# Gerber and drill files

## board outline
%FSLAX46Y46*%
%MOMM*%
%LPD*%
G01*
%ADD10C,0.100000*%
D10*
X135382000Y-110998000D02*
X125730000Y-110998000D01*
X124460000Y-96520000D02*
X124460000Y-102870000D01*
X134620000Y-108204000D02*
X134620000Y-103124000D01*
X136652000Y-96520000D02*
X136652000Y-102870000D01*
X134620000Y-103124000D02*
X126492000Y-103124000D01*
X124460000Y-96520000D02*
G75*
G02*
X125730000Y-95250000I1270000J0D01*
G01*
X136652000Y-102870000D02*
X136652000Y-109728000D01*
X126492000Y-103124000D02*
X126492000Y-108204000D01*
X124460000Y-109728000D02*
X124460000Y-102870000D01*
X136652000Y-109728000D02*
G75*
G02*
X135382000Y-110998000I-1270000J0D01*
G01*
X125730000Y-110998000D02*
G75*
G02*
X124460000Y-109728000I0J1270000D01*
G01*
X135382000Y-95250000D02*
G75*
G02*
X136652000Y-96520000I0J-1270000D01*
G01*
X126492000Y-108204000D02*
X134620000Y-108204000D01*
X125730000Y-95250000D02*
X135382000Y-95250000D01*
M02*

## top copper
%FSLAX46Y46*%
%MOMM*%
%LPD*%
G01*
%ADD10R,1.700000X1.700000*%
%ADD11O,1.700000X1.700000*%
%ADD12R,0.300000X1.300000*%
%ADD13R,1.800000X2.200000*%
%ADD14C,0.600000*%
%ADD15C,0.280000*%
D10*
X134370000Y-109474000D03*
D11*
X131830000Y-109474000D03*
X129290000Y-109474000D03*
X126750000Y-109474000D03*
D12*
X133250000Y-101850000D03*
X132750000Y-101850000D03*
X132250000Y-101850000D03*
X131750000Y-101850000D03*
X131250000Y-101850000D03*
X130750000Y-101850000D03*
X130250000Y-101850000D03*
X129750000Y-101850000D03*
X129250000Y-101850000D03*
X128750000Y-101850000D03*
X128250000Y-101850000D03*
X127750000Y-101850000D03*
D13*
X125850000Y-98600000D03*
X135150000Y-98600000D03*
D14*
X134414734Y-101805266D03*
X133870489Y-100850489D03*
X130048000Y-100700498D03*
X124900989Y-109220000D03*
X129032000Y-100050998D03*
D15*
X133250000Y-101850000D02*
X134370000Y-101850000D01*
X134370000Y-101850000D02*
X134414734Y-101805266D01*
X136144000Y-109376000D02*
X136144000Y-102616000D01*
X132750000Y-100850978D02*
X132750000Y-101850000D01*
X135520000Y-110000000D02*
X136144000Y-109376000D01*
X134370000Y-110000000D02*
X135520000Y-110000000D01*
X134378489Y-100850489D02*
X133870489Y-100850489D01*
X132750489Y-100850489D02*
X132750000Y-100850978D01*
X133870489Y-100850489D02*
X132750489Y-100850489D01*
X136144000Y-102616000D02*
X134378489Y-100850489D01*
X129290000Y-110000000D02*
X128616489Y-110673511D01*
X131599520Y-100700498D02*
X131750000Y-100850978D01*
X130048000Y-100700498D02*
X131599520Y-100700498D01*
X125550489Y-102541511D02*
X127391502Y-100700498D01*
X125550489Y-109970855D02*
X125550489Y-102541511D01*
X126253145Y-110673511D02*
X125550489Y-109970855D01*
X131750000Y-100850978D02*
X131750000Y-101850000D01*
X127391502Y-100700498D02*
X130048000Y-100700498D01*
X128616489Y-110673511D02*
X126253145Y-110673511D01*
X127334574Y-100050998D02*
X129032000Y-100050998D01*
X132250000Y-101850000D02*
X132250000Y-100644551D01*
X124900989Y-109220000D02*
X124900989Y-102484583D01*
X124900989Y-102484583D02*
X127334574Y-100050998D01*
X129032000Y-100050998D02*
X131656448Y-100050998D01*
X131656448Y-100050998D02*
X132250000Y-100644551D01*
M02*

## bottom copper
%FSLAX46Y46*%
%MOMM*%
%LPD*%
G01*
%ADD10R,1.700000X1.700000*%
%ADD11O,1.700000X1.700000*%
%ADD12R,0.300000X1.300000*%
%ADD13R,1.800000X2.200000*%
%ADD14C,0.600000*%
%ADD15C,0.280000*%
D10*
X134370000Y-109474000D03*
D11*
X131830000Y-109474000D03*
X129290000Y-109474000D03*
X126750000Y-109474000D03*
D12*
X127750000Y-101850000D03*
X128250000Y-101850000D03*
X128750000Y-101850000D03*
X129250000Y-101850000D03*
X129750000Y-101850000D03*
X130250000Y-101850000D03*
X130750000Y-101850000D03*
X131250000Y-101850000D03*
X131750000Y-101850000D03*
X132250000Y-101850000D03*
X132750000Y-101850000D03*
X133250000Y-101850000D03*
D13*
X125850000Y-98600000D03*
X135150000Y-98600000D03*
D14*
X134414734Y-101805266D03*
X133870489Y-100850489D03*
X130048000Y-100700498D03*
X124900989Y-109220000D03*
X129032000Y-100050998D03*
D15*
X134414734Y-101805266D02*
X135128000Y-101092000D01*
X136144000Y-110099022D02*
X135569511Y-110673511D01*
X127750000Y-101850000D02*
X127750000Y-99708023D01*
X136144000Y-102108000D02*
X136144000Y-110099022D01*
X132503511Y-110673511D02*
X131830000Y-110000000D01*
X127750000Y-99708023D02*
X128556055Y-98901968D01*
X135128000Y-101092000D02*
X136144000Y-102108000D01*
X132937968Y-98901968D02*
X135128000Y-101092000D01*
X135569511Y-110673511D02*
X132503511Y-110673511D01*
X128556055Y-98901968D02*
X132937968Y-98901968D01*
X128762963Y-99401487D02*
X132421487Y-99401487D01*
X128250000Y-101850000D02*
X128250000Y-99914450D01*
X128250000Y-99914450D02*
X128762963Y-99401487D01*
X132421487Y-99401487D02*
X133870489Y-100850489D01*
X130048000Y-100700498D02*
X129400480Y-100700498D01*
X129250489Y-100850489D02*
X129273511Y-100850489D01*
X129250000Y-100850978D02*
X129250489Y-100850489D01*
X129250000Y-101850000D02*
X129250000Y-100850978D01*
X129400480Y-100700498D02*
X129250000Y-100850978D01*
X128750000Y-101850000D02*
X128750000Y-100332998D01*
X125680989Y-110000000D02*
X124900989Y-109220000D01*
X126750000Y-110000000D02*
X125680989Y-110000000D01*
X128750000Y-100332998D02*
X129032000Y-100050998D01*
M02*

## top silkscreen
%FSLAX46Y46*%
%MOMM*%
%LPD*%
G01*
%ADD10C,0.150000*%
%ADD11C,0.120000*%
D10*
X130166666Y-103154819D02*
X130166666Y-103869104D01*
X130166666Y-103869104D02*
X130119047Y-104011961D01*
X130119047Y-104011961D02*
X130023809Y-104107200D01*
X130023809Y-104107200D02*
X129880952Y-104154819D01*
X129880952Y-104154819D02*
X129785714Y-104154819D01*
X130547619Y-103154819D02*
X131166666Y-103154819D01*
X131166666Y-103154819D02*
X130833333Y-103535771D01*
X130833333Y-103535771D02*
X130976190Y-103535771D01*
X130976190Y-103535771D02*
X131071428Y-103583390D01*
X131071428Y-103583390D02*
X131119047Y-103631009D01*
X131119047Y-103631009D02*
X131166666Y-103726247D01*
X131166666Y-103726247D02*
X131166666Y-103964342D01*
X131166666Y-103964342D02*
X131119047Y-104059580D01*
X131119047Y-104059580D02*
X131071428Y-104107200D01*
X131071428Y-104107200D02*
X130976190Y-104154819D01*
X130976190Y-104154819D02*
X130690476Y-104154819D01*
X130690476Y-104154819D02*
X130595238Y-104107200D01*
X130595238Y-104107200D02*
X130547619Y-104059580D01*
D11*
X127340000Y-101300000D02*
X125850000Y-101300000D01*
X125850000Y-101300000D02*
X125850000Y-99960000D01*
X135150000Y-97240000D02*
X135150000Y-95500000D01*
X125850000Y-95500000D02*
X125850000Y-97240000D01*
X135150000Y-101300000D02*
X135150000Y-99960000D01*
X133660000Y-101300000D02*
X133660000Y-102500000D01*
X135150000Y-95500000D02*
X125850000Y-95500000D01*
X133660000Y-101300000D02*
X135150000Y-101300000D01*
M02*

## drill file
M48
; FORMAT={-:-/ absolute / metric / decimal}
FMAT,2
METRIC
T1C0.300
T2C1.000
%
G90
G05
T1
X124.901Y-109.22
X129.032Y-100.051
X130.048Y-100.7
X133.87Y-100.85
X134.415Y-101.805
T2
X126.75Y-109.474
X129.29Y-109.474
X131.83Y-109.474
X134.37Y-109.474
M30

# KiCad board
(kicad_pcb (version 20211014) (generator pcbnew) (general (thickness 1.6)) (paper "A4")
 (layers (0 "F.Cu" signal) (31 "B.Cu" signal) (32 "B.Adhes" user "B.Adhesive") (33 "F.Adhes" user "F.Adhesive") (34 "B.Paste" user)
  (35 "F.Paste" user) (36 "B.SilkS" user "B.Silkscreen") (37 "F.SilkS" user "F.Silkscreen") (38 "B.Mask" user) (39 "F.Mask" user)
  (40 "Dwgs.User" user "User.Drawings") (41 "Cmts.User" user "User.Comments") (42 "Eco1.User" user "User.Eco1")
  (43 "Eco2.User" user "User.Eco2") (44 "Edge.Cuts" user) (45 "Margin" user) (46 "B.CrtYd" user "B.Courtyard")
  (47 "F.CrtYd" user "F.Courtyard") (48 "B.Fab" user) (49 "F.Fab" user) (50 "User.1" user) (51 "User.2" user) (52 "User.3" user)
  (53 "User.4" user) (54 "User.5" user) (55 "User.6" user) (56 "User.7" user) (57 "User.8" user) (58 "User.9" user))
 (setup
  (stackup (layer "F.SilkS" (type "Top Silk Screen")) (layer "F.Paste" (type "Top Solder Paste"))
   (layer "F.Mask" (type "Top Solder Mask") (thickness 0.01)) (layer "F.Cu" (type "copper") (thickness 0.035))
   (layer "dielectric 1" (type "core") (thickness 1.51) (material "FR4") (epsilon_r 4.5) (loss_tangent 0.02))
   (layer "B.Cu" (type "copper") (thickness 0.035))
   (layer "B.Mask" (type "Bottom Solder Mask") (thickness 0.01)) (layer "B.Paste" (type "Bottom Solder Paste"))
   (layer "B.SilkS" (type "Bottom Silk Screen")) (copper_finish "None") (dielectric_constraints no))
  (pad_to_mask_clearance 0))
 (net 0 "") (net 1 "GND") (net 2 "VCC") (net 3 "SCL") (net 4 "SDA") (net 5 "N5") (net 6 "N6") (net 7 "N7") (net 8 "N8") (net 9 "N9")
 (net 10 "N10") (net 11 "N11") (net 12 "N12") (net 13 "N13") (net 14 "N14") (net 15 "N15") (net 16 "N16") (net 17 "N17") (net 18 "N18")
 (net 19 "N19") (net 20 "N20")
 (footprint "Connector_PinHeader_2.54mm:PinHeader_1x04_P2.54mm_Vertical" (layer "F.Cu") (at 130.5 109.474 -90)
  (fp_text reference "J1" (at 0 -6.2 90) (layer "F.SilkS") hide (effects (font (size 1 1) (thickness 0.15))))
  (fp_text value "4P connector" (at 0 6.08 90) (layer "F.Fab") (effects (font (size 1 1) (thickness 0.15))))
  (pad "1" thru_hole rect (at 0 -3.87 270) (size 1.7 1.7) (drill 1) (layers *.Cu *.Mask) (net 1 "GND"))
  (pad "2" thru_hole oval (at 0 -1.33 270) (size 1.7 1.7) (drill 1) (layers *.Cu *.Mask) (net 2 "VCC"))
  (pad "3" thru_hole oval (at 0 1.21 270) (size 1.7 1.7) (drill 1) (layers *.Cu *.Mask) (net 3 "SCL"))
  (pad "4" thru_hole oval (at 0 3.75 270) (size 1.7 1.7) (drill 1) (layers *.Cu *.Mask) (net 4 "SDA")))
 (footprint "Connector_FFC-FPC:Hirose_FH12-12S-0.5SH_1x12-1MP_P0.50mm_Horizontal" (layer "F.Cu") (at 130.5 100 180)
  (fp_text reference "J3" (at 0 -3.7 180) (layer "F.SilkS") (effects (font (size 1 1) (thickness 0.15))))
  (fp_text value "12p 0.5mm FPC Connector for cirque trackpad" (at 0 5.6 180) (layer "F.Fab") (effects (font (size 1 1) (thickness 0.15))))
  (fp_line (start 3.16 -1.3) (end 4.65 -1.3) (layer "F.SilkS") (width 0.12))
  (fp_line (start 4.65 -1.3) (end 4.65 0.04) (layer "F.SilkS") (width 0.12))
  (fp_line (start -4.65 2.76) (end -4.65 4.5) (layer "F.SilkS") (width 0.12))
  (fp_line (start 4.65 4.5) (end 4.65 2.76) (layer "F.SilkS") (width 0.12))
  (fp_line (start -4.65 -1.3) (end -4.65 0.04) (layer "F.SilkS") (width 0.12))
  (fp_line (start -3.16 -1.3) (end -3.16 -2.5) (layer "F.SilkS") (width 0.12))
  (fp_line (start -4.65 4.5) (end 4.65 4.5) (layer "F.SilkS") (width 0.12))
  (fp_line (start -3.16 -1.3) (end -4.65 -1.3) (layer "F.SilkS") (width 0.12))
  (pad "1" smd rect (at -2.75 -1.85 180) (size 0.3 1.3) (layers "F.Cu" "F.Paste" "F.Mask") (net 2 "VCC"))
  (pad "2" smd rect (at -2.25 -1.85 180) (size 0.3 1.3) (layers "F.Cu" "F.Paste" "F.Mask") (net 1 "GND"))
  (pad "3" smd rect (at -1.75 -1.85 180) (size 0.3 1.3) (layers "F.Cu" "F.Paste" "F.Mask") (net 4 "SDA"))
  (pad "4" smd rect (at -1.25 -1.85 180) (size 0.3 1.3) (layers "F.Cu" "F.Paste" "F.Mask") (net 3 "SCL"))
  (pad "5" smd rect (at -0.75 -1.85 180) (size 0.3 1.3) (layers "F.Cu" "F.Paste" "F.Mask") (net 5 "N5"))
  (pad "6" smd rect (at -0.25 -1.85 180) (size 0.3 1.3) (layers "F.Cu" "F.Paste" "F.Mask") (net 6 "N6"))
  (pad "7" smd rect (at 0.25 -1.85 180) (size 0.3 1.3) (layers "F.Cu" "F.Paste" "F.Mask") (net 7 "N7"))
  (pad "8" smd rect (at 0.75 -1.85 180) (size 0.3 1.3) (layers "F.Cu" "F.Paste" "F.Mask") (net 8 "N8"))
  (pad "9" smd rect (at 1.25 -1.85 180) (size 0.3 1.3) (layers "F.Cu" "F.Paste" "F.Mask") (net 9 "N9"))
  (pad "10" smd rect (at 1.75 -1.85 180) (size 0.3 1.3) (layers "F.Cu" "F.Paste" "F.Mask") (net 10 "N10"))
  (pad "11" smd rect (at 2.25 -1.85 180) (size 0.3 1.3) (layers "F.Cu" "F.Paste" "F.Mask") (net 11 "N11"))
  (pad "12" smd rect (at 2.75 -1.85 180) (size 0.3 1.3) (layers "F.Cu" "F.Paste" "F.Mask") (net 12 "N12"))
  (pad "MP" smd rect (at 4.65 1.4 180) (size 1.8 2.2) (layers "F.Cu" "F.Paste" "F.Mask"))
  (pad "MP" smd rect (at -4.65 1.4 180) (size 1.8 2.2) (layers "F.Cu" "F.Paste" "F.Mask")))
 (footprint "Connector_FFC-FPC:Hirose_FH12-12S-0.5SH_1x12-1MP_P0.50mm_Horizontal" (layer "B.Cu") (at 130.5 100)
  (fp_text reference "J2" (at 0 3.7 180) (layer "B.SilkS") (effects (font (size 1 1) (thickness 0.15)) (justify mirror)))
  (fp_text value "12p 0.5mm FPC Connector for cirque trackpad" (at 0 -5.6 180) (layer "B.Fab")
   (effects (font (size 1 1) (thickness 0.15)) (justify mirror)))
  (pad "1" smd rect (at -2.75 1.85) (size 0.3 1.3) (layers "B.Cu" "B.Paste" "B.Mask") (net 2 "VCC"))
  (pad "2" smd rect (at -2.25 1.85) (size 0.3 1.3) (layers "B.Cu" "B.Paste" "B.Mask") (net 1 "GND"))
  (pad "3" smd rect (at -1.75 1.85) (size 0.3 1.3) (layers "B.Cu" "B.Paste" "B.Mask") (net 4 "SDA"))
  (pad "4" smd rect (at -1.25 1.85) (size 0.3 1.3) (layers "B.Cu" "B.Paste" "B.Mask") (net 3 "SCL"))
  (pad "5" smd rect (at -0.75 1.85) (size 0.3 1.3) (layers "B.Cu" "B.Paste" "B.Mask") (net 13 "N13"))
  (pad "6" smd rect (at -0.25 1.85) (size 0.3 1.3) (layers "B.Cu" "B.Paste" "B.Mask") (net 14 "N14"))
  (pad "7" smd rect (at 0.25 1.85) (size 0.3 1.3) (layers "B.Cu" "B.Paste" "B.Mask") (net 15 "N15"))
  (pad "8" smd rect (at 0.75 1.85) (size 0.3 1.3) (layers "B.Cu" "B.Paste" "B.Mask") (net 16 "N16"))
  (pad "9" smd rect (at 1.25 1.85) (size 0.3 1.3) (layers "B.Cu" "B.Paste" "B.Mask") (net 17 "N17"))
  (pad "10" smd rect (at 1.75 1.85) (size 0.3 1.3) (layers "B.Cu" "B.Paste" "B.Mask") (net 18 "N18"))
  (pad "11" smd rect (at 2.25 1.85) (size 0.3 1.3) (layers "B.Cu" "B.Paste" "B.Mask") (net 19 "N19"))
  (pad "12" smd rect (at 2.75 1.85) (size 0.3 1.3) (layers "B.Cu" "B.Paste" "B.Mask") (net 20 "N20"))
  (pad "MP" smd rect (at -4.65 -1.4) (size 1.8 2.2) (layers "B.Cu" "B.Paste" "B.Mask"))
  (pad "MP" smd rect (at 4.65 -1.4) (size 1.8 2.2) (layers "B.Cu" "B.Paste" "B.Mask")))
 (gr_line (start 135.382 110.998) (end 125.73 110.998) (layer "Edge.Cuts") (width 0.1))
 (gr_line (start 124.46 96.52) (end 124.46 102.87) (layer "Edge.Cuts") (width 0.1))
 (gr_line (start 134.62 108.204) (end 134.62 103.124) (layer "Edge.Cuts") (width 0.1))
 (gr_line (start 136.652 96.52) (end 136.652 102.87) (layer "Edge.Cuts") (width 0.1))
 (gr_line (start 134.62 103.124) (end 126.492 103.124) (layer "Edge.Cuts") (width 0.1))
 (gr_arc (start 124.46 96.52) (mid 124.831974 95.621974) (end 125.73 95.25) (layer "Edge.Cuts") (width 0.1))
 (gr_line (start 136.652 102.87) (end 136.652 109.728) (layer "Edge.Cuts") (width 0.1))
 (gr_line (start 126.492 103.124) (end 126.492 108.204) (layer "Edge.Cuts") (width 0.1))
 (gr_line (start 124.46 109.728) (end 124.46 102.87) (layer "Edge.Cuts") (width 0.1))
 (gr_arc (start 136.652 109.728) (mid 136.280026 110.626026) (end 135.382 110.998) (layer "Edge.Cuts") (width 0.1))
 (gr_arc (start 125.73 110.998) (mid 124.831974 110.626026) (end 124.46 109.728) (layer "Edge.Cuts") (width 0.1))
 (gr_arc (start 135.382 95.25) (mid 136.280026 95.621974) (end 136.652 96.52) (layer "Edge.Cuts") (width 0.1))
 (gr_line (start 126.492 108.204) (end 134.62 108.204) (layer "Edge.Cuts") (width 0.1))
 (gr_line (start 125.73 95.25) (end 135.382 95.25) (layer "Edge.Cuts") (width 0.1))
 (segment (start 133.25 101.85) (end 134.37 101.85) (width 0.28) (layer "F.Cu") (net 2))
 (segment (start 134.37 101.85) (end 134.414734 101.805266) (width 0.28) (layer "F.Cu") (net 2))
 (via (at 134.414734 101.805266) (size 0.6) (drill 0.3) (layers "F.Cu" "B.Cu") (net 2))
 (segment (start 134.414734 101.805266) (end 135.128 101.092) (width 0.28) (layer "B.Cu") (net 2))
 (segment (start 136.144 110.099022) (end 135.569511 110.673511) (width 0.28) (layer "B.Cu") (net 2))
 (segment (start 127.75 101.85) (end 127.75 99.708023) (width 0.28) (layer "B.Cu") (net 2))
 (segment (start 136.144 102.108) (end 136.144 110.099022) (width 0.28) (layer "B.Cu") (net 2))
 (segment (start 132.503511 110.673511) (end 131.83 110) (width 0.28) (layer "B.Cu") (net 2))
 (segment (start 127.75 99.708023) (end 128.556055 98.901968) (width 0.28) (layer "B.Cu") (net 2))
 (segment (start 135.128 101.092) (end 136.144 102.108) (width 0.28) (layer "B.Cu") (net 2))
 (segment (start 132.937968 98.901968) (end 135.128 101.092) (width 0.28) (layer "B.Cu") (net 2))
 (segment (start 135.569511 110.673511) (end 132.503511 110.673511) (width 0.28) (layer "B.Cu") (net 2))
 (segment (start 128.556055 98.901968) (end 132.937968 98.901968) (width 0.28) (layer "B.Cu") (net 2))
 (segment (start 136.144 109.376) (end 136.144 102.616) (width 0.28) (layer "F.Cu") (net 1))
 (segment (start 132.75 100.850978) (end 132.75 101.85) (width 0.28) (layer "F.Cu") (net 1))
 (segment (start 135.52 110) (end 136.144 109.376) (width 0.28) (layer "F.Cu") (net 1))
 (segment (start 134.37 110) (end 135.52 110) (width 0.28) (layer "F.Cu") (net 1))
 (segment (start 134.378489 100.850489) (end 133.870489 100.850489) (width 0.28) (layer "F.Cu") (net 1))
 (segment (start 132.750489 100.850489) (end 132.75 100.850978) (width 0.28) (layer "F.Cu") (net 1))
 (segment (start 133.870489 100.850489) (end 132.750489 100.850489) (width 0.28) (layer "F.Cu") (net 1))
 (segment (start 136.144 102.616) (end 134.378489 100.850489) (width 0.28) (layer "F.Cu") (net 1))
 (via (at 133.870489 100.850489) (size 0.6) (drill 0.3) (layers "F.Cu" "B.Cu") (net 1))
 (segment (start 128.762963 99.401487) (end 132.421487 99.401487) (width 0.28) (layer "B.Cu") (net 1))
 (segment (start 128.25 101.85) (end 128.25 99.91445) (width 0.28) (layer "B.Cu") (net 1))
 (segment (start 128.25 99.91445) (end 128.762963 99.401487) (width 0.28) (layer "B.Cu") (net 1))
 (segment (start 132.421487 99.401487) (end 133.870489 100.850489) (width 0.28) (layer "B.Cu") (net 1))
 (segment (start 129.29 110) (end 128.616489 110.673511) (width 0.28) (layer "F.Cu") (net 3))
 (segment (start 131.59952 100.700498) (end 131.75 100.850978) (width 0.28) (layer "F.Cu") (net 3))
 (segment (start 130.048 100.700498) (end 131.59952 100.700498) (width 0.28) (layer "F.Cu") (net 3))
 (segment (start 125.550489 102.541511) (end 127.391502 100.700498) (width 0.28) (layer "F.Cu") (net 3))
 (segment (start 125.550489 109.970855) (end 125.550489 102.541511) (width 0.28) (layer "F.Cu") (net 3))
 (segment (start 126.253145 110.673511) (end 125.550489 109.970855) (width 0.28) (layer "F.Cu") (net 3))
 (segment (start 131.75 100.850978) (end 131.75 101.85) (width 0.28) (layer "F.Cu") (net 3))
 (segment (start 127.391502 100.700498) (end 130.048 100.700498) (width 0.28) (layer "F.Cu") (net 3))
 (segment (start 128.616489 110.673511) (end 126.253145 110.673511) (width 0.28) (layer "F.Cu") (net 3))
 (via (at 130.048 100.700498) (size 0.6) (drill 0.3) (layers "F.Cu" "B.Cu") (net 3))
 (segment (start 130.048 100.700498) (end 129.40048 100.700498) (width 0.28) (layer "B.Cu") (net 3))
 (segment (start 129.250489 100.850489) (end 129.273511 100.850489) (width 0.28) (layer "B.Cu") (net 3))
 (segment (start 129.25 100.850978) (end 129.250489 100.850489) (width 0.28) (layer "B.Cu") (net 3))
 (segment (start 129.25 101.85) (end 129.25 100.850978) (width 0.28) (layer "B.Cu") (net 3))
 (segment (start 129.40048 100.700498) (end 129.25 100.850978) (width 0.28) (layer "B.Cu") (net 3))
 (segment (start 127.334574 100.050998) (end 129.032 100.050998) (width 0.28) (layer "F.Cu") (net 4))
 (segment (start 132.25 101.85) (end 132.25 100.644551) (width 0.28) (layer "F.Cu") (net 4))
 (segment (start 124.900989 109.22) (end 124.900989 102.484583) (width 0.28) (layer "F.Cu") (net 4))
 (segment (start 124.900989 102.484583) (end 127.334574 100.050998) (width 0.28) (layer "F.Cu") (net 4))
 (segment (start 129.032 100.050998) (end 131.656448 100.050998) (width 0.28) (layer "F.Cu") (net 4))
 (segment (start 131.656448 100.050998) (end 132.25 100.644551) (width 0.28) (layer "F.Cu") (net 4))
 (via (at 124.900989 109.22) (size 0.6) (drill 0.3) (layers "F.Cu" "B.Cu") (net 4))
 (via (at 129.032 100.050998) (size 0.6) (drill 0.3) (layers "F.Cu" "B.Cu") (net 4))
 (segment (start 128.75 101.85) (end 128.75 100.332998) (width 0.28) (layer "B.Cu") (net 4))
 (segment (start 125.680989 110) (end 124.900989 109.22) (width 0.28) (layer "B.Cu") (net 4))
 (segment (start 126.75 110) (end 125.680989 110) (width 0.28) (layer "B.Cu") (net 4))
 (segment (start 128.75 100.332998) (end 129.032 100.050998) (width 0.28) (layer "B.Cu") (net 4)))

